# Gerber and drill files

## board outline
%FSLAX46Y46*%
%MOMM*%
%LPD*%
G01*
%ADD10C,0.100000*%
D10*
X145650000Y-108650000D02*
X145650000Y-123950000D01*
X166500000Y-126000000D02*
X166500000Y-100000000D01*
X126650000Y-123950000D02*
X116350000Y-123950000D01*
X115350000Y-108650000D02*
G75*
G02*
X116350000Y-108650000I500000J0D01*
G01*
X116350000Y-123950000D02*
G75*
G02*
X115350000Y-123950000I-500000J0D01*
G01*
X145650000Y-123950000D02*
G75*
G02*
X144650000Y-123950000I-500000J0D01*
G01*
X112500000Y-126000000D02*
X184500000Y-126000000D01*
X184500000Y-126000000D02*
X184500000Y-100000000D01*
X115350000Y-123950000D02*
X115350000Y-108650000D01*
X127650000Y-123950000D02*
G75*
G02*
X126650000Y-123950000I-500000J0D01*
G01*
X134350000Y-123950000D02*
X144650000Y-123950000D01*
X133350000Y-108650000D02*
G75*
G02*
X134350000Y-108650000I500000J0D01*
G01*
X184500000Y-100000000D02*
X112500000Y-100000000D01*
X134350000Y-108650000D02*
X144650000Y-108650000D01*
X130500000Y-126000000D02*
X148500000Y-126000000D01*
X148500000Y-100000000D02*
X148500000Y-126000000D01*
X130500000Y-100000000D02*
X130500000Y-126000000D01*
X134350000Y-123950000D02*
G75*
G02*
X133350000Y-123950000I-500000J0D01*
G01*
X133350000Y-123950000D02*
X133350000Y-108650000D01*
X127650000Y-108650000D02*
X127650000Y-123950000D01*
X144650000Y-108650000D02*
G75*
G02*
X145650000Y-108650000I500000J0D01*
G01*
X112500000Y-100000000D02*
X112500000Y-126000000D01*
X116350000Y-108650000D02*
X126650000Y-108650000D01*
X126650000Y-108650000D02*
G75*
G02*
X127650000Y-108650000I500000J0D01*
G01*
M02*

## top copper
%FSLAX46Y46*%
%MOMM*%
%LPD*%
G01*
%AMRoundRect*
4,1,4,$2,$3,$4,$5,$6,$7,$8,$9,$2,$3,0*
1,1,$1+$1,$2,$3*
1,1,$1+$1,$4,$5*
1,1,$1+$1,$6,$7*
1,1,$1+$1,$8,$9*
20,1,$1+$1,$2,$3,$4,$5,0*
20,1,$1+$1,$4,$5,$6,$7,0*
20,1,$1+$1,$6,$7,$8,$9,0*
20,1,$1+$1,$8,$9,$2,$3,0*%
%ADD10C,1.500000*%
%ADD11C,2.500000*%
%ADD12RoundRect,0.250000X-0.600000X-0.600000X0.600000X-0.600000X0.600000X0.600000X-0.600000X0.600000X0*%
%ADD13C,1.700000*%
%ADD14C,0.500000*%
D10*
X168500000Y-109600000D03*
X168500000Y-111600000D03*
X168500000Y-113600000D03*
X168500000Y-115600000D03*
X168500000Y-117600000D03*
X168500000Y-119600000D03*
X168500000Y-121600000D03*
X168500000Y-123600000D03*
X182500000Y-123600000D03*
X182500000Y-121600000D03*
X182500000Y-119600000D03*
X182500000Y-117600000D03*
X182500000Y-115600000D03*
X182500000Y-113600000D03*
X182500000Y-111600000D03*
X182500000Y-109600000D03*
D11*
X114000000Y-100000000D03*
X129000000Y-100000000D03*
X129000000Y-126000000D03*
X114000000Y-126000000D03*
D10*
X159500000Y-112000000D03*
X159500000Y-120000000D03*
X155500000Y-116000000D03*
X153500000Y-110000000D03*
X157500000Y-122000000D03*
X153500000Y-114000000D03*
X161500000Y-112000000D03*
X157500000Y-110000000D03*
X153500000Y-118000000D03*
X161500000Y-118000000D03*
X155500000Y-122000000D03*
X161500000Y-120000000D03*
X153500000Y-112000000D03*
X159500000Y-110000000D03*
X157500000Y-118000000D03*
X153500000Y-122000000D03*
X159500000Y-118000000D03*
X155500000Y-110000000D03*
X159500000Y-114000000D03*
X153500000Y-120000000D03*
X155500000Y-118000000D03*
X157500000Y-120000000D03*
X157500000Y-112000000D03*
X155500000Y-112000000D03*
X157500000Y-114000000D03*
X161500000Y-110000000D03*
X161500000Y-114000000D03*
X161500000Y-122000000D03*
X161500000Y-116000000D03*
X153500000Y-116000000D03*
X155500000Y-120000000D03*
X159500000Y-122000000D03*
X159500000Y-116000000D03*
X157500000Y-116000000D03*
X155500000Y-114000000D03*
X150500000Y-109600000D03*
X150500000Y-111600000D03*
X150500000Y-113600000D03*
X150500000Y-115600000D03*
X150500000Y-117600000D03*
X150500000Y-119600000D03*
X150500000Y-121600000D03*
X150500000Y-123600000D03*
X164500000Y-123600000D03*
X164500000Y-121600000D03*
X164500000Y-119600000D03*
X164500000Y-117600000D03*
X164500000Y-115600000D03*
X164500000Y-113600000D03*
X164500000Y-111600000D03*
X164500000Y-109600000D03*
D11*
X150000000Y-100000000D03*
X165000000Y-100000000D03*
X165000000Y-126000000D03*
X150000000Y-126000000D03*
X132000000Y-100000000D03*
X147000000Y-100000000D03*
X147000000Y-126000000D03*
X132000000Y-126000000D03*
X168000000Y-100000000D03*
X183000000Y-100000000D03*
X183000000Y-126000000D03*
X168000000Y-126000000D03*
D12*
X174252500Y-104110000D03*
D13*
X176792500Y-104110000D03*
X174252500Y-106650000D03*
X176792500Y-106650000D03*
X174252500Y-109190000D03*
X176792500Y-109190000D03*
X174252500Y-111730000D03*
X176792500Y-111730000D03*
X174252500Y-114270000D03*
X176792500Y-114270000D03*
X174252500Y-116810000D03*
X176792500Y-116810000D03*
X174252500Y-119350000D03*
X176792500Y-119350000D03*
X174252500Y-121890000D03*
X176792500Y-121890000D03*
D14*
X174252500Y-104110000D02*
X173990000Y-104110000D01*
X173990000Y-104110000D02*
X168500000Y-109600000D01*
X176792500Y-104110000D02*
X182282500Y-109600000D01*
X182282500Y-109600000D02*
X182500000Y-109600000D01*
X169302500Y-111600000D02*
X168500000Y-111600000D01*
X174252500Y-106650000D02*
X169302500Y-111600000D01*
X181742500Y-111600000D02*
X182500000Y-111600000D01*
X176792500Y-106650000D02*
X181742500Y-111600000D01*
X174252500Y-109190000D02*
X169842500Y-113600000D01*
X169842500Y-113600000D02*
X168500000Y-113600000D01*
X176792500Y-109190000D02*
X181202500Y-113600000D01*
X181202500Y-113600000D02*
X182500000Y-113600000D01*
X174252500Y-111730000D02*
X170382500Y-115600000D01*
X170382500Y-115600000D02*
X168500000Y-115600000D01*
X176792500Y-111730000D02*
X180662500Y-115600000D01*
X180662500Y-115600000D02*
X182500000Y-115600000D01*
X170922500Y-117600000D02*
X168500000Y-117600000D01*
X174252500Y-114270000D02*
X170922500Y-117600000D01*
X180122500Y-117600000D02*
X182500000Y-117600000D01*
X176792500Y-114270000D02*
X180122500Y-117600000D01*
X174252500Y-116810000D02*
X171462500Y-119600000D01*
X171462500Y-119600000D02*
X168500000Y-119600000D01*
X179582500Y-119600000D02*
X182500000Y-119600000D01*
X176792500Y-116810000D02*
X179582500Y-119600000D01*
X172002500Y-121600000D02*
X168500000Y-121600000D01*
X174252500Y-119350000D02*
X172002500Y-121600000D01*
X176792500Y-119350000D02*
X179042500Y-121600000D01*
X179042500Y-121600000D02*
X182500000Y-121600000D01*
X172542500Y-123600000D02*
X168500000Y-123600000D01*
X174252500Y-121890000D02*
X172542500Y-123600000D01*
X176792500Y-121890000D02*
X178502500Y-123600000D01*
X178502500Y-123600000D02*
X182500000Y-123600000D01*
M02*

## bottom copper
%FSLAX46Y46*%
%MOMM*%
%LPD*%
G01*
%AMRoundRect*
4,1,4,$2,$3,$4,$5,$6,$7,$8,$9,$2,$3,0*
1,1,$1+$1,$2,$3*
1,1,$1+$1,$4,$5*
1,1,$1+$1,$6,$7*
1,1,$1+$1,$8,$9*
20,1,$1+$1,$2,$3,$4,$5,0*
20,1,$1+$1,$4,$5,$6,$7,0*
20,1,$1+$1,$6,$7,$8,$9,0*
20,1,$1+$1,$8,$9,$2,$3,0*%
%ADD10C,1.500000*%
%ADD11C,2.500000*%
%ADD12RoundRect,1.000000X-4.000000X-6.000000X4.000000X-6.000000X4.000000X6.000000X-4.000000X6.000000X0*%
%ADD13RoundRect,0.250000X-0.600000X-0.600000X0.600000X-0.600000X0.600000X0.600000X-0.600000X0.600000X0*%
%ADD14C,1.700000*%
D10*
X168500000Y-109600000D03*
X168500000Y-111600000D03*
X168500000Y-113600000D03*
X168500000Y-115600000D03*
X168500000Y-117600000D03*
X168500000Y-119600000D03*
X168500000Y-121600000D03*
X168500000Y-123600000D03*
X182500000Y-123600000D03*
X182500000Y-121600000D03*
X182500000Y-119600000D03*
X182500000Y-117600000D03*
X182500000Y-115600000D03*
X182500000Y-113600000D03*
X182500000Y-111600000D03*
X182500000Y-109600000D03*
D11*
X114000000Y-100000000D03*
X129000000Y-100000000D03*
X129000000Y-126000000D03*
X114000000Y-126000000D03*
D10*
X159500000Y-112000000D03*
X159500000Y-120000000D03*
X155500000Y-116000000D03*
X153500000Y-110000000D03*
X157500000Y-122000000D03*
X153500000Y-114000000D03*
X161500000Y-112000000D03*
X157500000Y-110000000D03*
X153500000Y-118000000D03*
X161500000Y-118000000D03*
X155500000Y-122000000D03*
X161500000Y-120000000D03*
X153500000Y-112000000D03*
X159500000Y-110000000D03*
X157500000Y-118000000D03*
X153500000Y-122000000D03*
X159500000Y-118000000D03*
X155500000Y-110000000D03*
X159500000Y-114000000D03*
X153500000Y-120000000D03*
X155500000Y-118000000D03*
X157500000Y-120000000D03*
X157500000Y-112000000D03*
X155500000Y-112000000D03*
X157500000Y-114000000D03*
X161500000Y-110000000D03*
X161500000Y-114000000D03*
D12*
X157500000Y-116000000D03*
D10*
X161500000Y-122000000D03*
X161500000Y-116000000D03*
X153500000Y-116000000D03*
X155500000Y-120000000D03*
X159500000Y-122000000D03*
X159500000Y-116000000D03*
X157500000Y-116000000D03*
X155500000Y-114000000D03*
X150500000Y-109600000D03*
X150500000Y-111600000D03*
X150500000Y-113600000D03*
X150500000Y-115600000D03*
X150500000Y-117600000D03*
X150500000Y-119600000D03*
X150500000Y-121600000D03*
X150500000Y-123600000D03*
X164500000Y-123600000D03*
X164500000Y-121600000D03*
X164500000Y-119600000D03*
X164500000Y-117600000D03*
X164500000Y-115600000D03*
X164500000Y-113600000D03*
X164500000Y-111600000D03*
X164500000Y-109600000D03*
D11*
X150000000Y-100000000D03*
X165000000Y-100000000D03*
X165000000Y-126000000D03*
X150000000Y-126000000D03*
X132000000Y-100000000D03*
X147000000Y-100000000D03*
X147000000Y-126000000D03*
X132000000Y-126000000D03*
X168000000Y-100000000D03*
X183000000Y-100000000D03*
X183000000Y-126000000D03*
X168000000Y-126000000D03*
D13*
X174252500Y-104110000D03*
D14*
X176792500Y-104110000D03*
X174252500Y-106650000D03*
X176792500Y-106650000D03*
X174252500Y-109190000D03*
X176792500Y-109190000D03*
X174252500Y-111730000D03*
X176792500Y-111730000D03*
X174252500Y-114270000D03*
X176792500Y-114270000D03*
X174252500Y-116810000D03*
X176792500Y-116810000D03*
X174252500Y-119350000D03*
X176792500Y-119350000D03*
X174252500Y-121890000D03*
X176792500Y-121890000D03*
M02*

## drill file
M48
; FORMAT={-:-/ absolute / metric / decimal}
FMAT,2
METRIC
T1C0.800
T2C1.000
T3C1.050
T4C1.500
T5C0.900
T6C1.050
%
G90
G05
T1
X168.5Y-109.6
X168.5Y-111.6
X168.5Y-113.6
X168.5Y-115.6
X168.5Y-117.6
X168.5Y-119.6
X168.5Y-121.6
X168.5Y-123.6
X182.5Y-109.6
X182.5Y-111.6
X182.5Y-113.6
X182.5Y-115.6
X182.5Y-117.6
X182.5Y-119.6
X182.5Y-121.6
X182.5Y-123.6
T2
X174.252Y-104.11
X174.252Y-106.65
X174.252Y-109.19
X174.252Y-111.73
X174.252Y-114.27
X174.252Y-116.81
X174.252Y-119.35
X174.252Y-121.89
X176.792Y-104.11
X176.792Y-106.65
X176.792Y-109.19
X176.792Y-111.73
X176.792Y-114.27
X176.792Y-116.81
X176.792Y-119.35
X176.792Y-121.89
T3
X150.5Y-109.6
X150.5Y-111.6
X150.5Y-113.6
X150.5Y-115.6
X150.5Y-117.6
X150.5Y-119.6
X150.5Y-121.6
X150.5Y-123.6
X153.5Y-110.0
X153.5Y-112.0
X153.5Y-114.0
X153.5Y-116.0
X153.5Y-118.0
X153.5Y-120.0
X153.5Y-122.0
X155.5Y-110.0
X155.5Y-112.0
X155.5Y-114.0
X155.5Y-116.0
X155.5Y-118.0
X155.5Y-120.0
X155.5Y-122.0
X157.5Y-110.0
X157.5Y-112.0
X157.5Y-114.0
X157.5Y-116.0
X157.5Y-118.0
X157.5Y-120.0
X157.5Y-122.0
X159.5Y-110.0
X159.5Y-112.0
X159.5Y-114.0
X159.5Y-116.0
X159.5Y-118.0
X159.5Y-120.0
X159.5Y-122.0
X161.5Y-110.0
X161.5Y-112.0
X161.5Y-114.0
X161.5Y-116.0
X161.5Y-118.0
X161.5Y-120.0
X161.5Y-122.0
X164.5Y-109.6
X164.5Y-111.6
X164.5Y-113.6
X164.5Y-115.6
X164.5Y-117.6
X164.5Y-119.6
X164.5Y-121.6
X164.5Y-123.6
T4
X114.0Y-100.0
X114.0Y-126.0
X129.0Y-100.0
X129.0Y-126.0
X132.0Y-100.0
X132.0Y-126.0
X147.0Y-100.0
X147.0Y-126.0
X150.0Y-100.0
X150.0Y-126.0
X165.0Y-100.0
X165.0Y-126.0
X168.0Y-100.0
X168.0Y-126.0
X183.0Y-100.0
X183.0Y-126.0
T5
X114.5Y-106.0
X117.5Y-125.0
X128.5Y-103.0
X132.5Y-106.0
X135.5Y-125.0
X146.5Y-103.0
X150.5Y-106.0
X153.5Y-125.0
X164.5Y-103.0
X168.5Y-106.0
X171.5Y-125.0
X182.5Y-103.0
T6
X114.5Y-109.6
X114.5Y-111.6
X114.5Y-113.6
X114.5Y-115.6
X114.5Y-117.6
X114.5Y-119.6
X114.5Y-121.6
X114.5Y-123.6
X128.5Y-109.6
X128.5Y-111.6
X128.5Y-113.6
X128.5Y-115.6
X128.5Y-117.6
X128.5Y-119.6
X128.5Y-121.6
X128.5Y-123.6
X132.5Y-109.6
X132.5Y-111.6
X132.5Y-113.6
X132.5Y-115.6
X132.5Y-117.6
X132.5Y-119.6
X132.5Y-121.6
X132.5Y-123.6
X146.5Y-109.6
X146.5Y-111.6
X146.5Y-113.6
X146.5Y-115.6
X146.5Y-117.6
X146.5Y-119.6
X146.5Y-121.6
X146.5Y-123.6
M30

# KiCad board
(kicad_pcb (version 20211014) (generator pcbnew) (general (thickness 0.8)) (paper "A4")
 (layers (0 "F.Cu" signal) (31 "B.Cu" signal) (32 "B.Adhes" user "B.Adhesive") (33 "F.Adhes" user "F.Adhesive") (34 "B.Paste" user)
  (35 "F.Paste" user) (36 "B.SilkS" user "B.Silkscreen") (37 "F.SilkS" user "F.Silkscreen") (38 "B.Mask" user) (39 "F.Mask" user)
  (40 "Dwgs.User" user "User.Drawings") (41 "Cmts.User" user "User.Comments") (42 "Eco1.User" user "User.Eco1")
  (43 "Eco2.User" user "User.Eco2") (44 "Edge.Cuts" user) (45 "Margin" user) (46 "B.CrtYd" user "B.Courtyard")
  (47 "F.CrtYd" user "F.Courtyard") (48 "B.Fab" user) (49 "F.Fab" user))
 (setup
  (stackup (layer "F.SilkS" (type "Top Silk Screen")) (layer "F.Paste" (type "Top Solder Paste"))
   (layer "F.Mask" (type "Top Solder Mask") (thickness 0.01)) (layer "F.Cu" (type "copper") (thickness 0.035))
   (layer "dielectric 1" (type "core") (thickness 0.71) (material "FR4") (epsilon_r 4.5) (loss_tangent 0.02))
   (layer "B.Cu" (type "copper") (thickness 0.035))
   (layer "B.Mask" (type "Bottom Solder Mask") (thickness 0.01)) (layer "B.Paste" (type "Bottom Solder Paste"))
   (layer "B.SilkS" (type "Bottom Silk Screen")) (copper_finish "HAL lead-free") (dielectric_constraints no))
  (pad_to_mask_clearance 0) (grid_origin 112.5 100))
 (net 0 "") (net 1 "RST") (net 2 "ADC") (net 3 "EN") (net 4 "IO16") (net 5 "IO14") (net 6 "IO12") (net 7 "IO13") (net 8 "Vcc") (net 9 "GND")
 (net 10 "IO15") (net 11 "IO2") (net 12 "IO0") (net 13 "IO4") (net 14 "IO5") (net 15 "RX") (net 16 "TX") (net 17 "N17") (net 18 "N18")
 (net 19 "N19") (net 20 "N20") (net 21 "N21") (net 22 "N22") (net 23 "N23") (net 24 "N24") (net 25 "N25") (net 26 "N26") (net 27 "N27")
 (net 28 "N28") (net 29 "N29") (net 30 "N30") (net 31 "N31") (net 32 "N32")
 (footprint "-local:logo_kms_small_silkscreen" (layer "F.Cu") (at 153 104.474422)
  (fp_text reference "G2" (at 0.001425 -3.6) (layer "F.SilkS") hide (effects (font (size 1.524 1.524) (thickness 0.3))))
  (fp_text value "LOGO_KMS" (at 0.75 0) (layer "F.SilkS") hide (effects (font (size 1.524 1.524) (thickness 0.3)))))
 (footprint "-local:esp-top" (layer "F.Cu") (at 166.5 100)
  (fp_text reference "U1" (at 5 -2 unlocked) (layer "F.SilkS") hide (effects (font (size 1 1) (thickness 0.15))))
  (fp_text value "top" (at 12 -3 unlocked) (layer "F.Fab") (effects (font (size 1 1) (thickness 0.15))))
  (pad "1" thru_hole circle (at 2 9.6) (size 1.5 1.5) (drill 0.8) (layers *.Cu *.Mask) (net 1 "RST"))
  (pad "2" thru_hole circle (at 2 11.6) (size 1.5 1.5) (drill 0.8) (layers *.Cu *.Mask) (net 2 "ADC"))
  (pad "3" thru_hole circle (at 2 13.6) (size 1.5 1.5) (drill 0.8) (layers *.Cu *.Mask) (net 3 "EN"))
  (pad "4" thru_hole circle (at 2 15.6) (size 1.5 1.5) (drill 0.8) (layers *.Cu *.Mask) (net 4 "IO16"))
  (pad "5" thru_hole circle (at 2 17.6) (size 1.5 1.5) (drill 0.8) (layers *.Cu *.Mask) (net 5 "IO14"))
  (pad "6" thru_hole circle (at 2 19.6) (size 1.5 1.5) (drill 0.8) (layers *.Cu *.Mask) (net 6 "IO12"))
  (pad "7" thru_hole circle (at 2 21.6) (size 1.5 1.5) (drill 0.8) (layers *.Cu *.Mask) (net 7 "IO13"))
  (pad "8" thru_hole circle (at 2 23.6) (size 1.5 1.5) (drill 0.8) (layers *.Cu *.Mask) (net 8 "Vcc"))
  (pad "9" thru_hole circle (at 16 23.6) (size 1.5 1.5) (drill 0.8) (layers *.Cu *.Mask) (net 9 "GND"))
  (pad "10" thru_hole circle (at 16 21.6) (size 1.5 1.5) (drill 0.8) (layers *.Cu *.Mask) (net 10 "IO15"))
  (pad "11" thru_hole circle (at 16 19.6) (size 1.5 1.5) (drill 0.8) (layers *.Cu *.Mask) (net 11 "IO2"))
  (pad "12" thru_hole circle (at 16 17.6) (size 1.5 1.5) (drill 0.8) (layers *.Cu *.Mask) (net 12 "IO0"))
  (pad "13" thru_hole circle (at 16 15.6) (size 1.5 1.5) (drill 0.8) (layers *.Cu *.Mask) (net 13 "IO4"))
  (pad "14" thru_hole circle (at 16 13.6) (size 1.5 1.5) (drill 0.8) (layers *.Cu *.Mask) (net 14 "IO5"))
  (pad "15" thru_hole circle (at 16 11.6) (size 1.5 1.5) (drill 0.8) (layers *.Cu *.Mask) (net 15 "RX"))
  (pad "16" thru_hole circle (at 16 9.6) (size 1.5 1.5) (drill 0.8) (layers *.Cu *.Mask) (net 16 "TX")))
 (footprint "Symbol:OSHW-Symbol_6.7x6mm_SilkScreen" (layer "F.Cu") (at 161 104.5)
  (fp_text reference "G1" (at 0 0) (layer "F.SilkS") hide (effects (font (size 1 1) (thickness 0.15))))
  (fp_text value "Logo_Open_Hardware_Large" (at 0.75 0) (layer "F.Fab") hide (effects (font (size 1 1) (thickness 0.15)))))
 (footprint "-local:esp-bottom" (layer "F.Cu") (at 112.5 100)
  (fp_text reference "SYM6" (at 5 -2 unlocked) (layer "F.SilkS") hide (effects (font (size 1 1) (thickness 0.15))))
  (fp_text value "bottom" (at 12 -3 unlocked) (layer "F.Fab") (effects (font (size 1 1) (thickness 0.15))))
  (pad "" np_thru_hole circle (at 2 23.6) (size 1.05 1.05) (drill 1.05) (layers F&B.Cu *.Mask))
  (pad "" np_thru_hole circle (at 16 19.6) (size 1.05 1.05) (drill 1.05) (layers F&B.Cu *.Mask))
  (pad "" np_thru_hole circle (at 2 13.6) (size 1.05 1.05) (drill 1.05) (layers F&B.Cu *.Mask))
  (pad "" np_thru_hole circle (at 2 11.6) (size 1.05 1.05) (drill 1.05) (layers F&B.Cu *.Mask))
  (pad "" np_thru_hole circle (at 2 15.6) (size 1.05 1.05) (drill 1.05) (layers F&B.Cu *.Mask))
  (pad "" np_thru_hole circle (at 16 9.6) (size 1.05 1.05) (drill 1.05) (layers F&B.Cu *.Mask))
  (pad "" np_thru_hole circle (at 2 9.6) (size 1.05 1.05) (drill 1.05) (layers F&B.Cu *.Mask))
  (pad "" np_thru_hole circle (at 16 23.6) (size 1.05 1.05) (drill 1.05) (layers F&B.Cu *.Mask))
  (pad "" np_thru_hole circle (at 2 17.6) (size 1.05 1.05) (drill 1.05) (layers F&B.Cu *.Mask))
  (pad "" np_thru_hole circle (at 16 13.6) (size 1.05 1.05) (drill 1.05) (layers F&B.Cu *.Mask))
  (pad "" np_thru_hole circle (at 2 19.6) (size 1.05 1.05) (drill 1.05) (layers F&B.Cu *.Mask))
  (pad "" np_thru_hole circle (at 16 17.6) (size 1.05 1.05) (drill 1.05) (layers F&B.Cu *.Mask))
  (pad "" np_thru_hole circle (at 16 11.6) (size 1.05 1.05) (drill 1.05) (layers F&B.Cu *.Mask))
  (pad "" np_thru_hole circle (at 16 21.6) (size 1.05 1.05) (drill 1.05) (layers F&B.Cu *.Mask))
  (pad "" np_thru_hole circle (at 2 21.6) (size 1.05 1.05) (drill 1.05) (layers F&B.Cu *.Mask))
  (pad "" np_thru_hole circle (at 16 15.6) (size 1.05 1.05) (drill 1.05) (layers F&B.Cu *.Mask)))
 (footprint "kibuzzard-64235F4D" (layer "F.Cu") (at 157.5 124.5)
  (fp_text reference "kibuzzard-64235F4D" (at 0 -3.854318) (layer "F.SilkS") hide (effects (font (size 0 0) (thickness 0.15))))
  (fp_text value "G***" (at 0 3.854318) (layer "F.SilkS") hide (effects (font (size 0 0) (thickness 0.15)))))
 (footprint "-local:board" (layer "F.Cu") (at 112.5 100)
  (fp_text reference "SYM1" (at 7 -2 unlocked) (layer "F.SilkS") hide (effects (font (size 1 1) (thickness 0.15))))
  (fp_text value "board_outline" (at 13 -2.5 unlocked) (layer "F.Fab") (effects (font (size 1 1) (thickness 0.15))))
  (pad "" np_thru_hole circle (at 16 3) (size 0.9 0.9) (drill 0.9) (layers F&B.Cu *.Mask))
  (pad "" np_thru_hole circle (at 5 25) (size 0.9 0.9) (drill 0.9) (layers F&B.Cu *.Mask))
  (pad "" np_thru_hole circle (at 2 6) (size 0.9 0.9) (drill 0.9) (layers F&B.Cu *.Mask))
  (pad "1" thru_hole circle (at 1.5 0) (size 2.5 2.5) (drill 1.5) (layers *.Cu *.Mask))
  (pad "2" thru_hole circle (at 16.5 0) (size 2.5 2.5) (drill 1.5) (layers *.Cu *.Mask))
  (pad "3" thru_hole circle (at 16.5 26) (size 2.5 2.5) (drill 1.5) (layers *.Cu *.Mask))
  (pad "4" thru_hole circle (at 1.5 26) (size 2.5 2.5) (drill 1.5) (layers *.Cu *.Mask)))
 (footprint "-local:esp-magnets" (layer "F.Cu") (at 148.5 100)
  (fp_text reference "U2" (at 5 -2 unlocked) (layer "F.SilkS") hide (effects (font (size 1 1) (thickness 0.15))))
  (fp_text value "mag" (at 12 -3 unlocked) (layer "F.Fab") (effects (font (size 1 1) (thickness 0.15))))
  (pad "" thru_hole circle (at 11 12) (size 1.5 1.5) (drill 1.05) (layers *.Cu *.Mask))
  (pad "" thru_hole circle (at 11 20) (size 1.5 1.5) (drill 1.05) (layers *.Cu *.Mask))
  (pad "" thru_hole circle (at 7 16) (size 1.5 1.5) (drill 1.05) (layers *.Cu *.Mask))
  (pad "" thru_hole circle (at 5 10) (size 1.5 1.5) (drill 1.05) (layers *.Cu *.Mask))
  (pad "" thru_hole circle (at 9 22) (size 1.5 1.5) (drill 1.05) (layers *.Cu *.Mask))
  (pad "" thru_hole circle (at 5 14) (size 1.5 1.5) (drill 1.05) (layers *.Cu *.Mask))
  (pad "" thru_hole circle (at 13 12) (size 1.5 1.5) (drill 1.05) (layers *.Cu *.Mask))
  (pad "" thru_hole circle (at 9 10) (size 1.5 1.5) (drill 1.05) (layers *.Cu *.Mask))
  (pad "" thru_hole circle (at 5 18) (size 1.5 1.5) (drill 1.05) (layers *.Cu *.Mask))
  (pad "" thru_hole circle (at 13 18) (size 1.5 1.5) (drill 1.05) (layers *.Cu *.Mask))
  (pad "" thru_hole circle (at 7 22) (size 1.5 1.5) (drill 1.05) (layers *.Cu *.Mask))
  (pad "" thru_hole circle (at 13 20) (size 1.5 1.5) (drill 1.05) (layers *.Cu *.Mask))
  (pad "" thru_hole circle (at 5 12) (size 1.5 1.5) (drill 1.05) (layers *.Cu *.Mask))
  (pad "" thru_hole circle (at 11 10) (size 1.5 1.5) (drill 1.05) (layers *.Cu *.Mask))
  (pad "" thru_hole circle (at 9 18) (size 1.5 1.5) (drill 1.05) (layers *.Cu *.Mask))
  (pad "" thru_hole circle (at 5 22) (size 1.5 1.5) (drill 1.05) (layers *.Cu *.Mask))
  (pad "" thru_hole circle (at 11 18) (size 1.5 1.5) (drill 1.05) (layers *.Cu *.Mask))
  (pad "" thru_hole circle (at 7 10) (size 1.5 1.5) (drill 1.05) (layers *.Cu *.Mask))
  (pad "" thru_hole circle (at 11 14) (size 1.5 1.5) (drill 1.05) (layers *.Cu *.Mask))
  (pad "" thru_hole circle (at 5 20) (size 1.5 1.5) (drill 1.05) (layers *.Cu *.Mask))
  (pad "" thru_hole circle (at 7 18) (size 1.5 1.5) (drill 1.05) (layers *.Cu *.Mask))
  (pad "" thru_hole circle (at 9 20) (size 1.5 1.5) (drill 1.05) (layers *.Cu *.Mask))
  (pad "" thru_hole circle (at 9 12) (size 1.5 1.5) (drill 1.05) (layers *.Cu *.Mask))
  (pad "" thru_hole circle (at 7 12) (size 1.5 1.5) (drill 1.05) (layers *.Cu *.Mask))
  (pad "" thru_hole circle (at 9 14) (size 1.5 1.5) (drill 1.05) (layers *.Cu *.Mask))
  (pad "" thru_hole circle (at 13 10) (size 1.5 1.5) (drill 1.05) (layers *.Cu *.Mask))
  (pad "" thru_hole circle (at 13 14) (size 1.5 1.5) (drill 1.05) (layers *.Cu *.Mask))
  (pad "" smd roundrect (at 9 16) (size 10 14) (layers "B.Cu" "B.Mask") (roundrect_rratio 0.1))
  (pad "" thru_hole circle (at 13 22) (size 1.5 1.5) (drill 1.05) (layers *.Cu *.Mask))
  (pad "" thru_hole circle (at 13 16) (size 1.5 1.5) (drill 1.05) (layers *.Cu *.Mask))
  (pad "" thru_hole circle (at 5 16) (size 1.5 1.5) (drill 1.05) (layers *.Cu *.Mask))
  (pad "" thru_hole circle (at 7 20) (size 1.5 1.5) (drill 1.05) (layers *.Cu *.Mask))
  (pad "" thru_hole circle (at 11 22) (size 1.5 1.5) (drill 1.05) (layers *.Cu *.Mask))
  (pad "" thru_hole circle (at 11 16) (size 1.5 1.5) (drill 1.05) (layers *.Cu *.Mask))
  (pad "" thru_hole circle (at 9 16) (size 1.5 1.5) (drill 1.05) (layers *.Cu *.Mask))
  (pad "" thru_hole circle (at 7 14) (size 1.5 1.5) (drill 1.05) (layers *.Cu *.Mask))
  (pad "1" thru_hole circle (at 2 9.6) (size 1.5 1.5) (drill 1.05) (layers *.Cu *.Mask) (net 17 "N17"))
  (pad "2" thru_hole circle (at 2 11.6) (size 1.5 1.5) (drill 1.05) (layers *.Cu *.Mask) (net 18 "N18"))
  (pad "3" thru_hole circle (at 2 13.6) (size 1.5 1.5) (drill 1.05) (layers *.Cu *.Mask) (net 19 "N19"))
  (pad "4" thru_hole circle (at 2 15.6) (size 1.5 1.5) (drill 1.05) (layers *.Cu *.Mask) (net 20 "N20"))
  (pad "5" thru_hole circle (at 2 17.6) (size 1.5 1.5) (drill 1.05) (layers *.Cu *.Mask) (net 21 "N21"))
  (pad "6" thru_hole circle (at 2 19.6) (size 1.5 1.5) (drill 1.05) (layers *.Cu *.Mask) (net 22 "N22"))
  (pad "7" thru_hole circle (at 2 21.6) (size 1.5 1.5) (drill 1.05) (layers *.Cu *.Mask) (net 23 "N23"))
  (pad "8" thru_hole circle (at 2 23.6) (size 1.5 1.5) (drill 1.05) (layers *.Cu *.Mask) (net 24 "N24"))
  (pad "9" thru_hole circle (at 16 23.6) (size 1.5 1.5) (drill 1.05) (layers *.Cu *.Mask) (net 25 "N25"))
  (pad "10" thru_hole circle (at 16 21.6) (size 1.5 1.5) (drill 1.05) (layers *.Cu *.Mask) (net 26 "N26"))
  (pad "11" thru_hole circle (at 16 19.6) (size 1.5 1.5) (drill 1.05) (layers *.Cu *.Mask) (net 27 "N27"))
  (pad "12" thru_hole circle (at 16 17.6) (size 1.5 1.5) (drill 1.05) (layers *.Cu *.Mask) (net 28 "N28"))
  (pad "13" thru_hole circle (at 16 15.6) (size 1.5 1.5) (drill 1.05) (layers *.Cu *.Mask) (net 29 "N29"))
  (pad "14" thru_hole circle (at 16 13.6) (size 1.5 1.5) (drill 1.05) (layers *.Cu *.Mask) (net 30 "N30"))
  (pad "15" thru_hole circle (at 16 11.6) (size 1.5 1.5) (drill 1.05) (layers *.Cu *.Mask) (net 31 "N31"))
  (pad "16" thru_hole circle (at 16 9.6) (size 1.5 1.5) (drill 1.05) (layers *.Cu *.Mask) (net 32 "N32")))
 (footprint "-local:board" (layer "F.Cu") (at 148.5 100)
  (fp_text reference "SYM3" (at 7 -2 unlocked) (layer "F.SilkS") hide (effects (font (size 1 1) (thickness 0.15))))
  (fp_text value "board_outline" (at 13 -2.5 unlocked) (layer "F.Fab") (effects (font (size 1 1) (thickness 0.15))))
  (pad "" np_thru_hole circle (at 5 25) (size 0.9 0.9) (drill 0.9) (layers F&B.Cu *.Mask))
  (pad "" np_thru_hole circle (at 2 6) (size 0.9 0.9) (drill 0.9) (layers F&B.Cu *.Mask))
  (pad "" np_thru_hole circle (at 16 3) (size 0.9 0.9) (drill 0.9) (layers F&B.Cu *.Mask))
  (pad "1" thru_hole circle (at 1.5 0) (size 2.5 2.5) (drill 1.5) (layers *.Cu *.Mask))
  (pad "2" thru_hole circle (at 16.5 0) (size 2.5 2.5) (drill 1.5) (layers *.Cu *.Mask))
  (pad "3" thru_hole circle (at 16.5 26) (size 2.5 2.5) (drill 1.5) (layers *.Cu *.Mask))
  (pad "4" thru_hole circle (at 1.5 26) (size 2.5 2.5) (drill 1.5) (layers *.Cu *.Mask)))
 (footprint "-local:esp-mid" (layer "F.Cu") (at 130.5 100)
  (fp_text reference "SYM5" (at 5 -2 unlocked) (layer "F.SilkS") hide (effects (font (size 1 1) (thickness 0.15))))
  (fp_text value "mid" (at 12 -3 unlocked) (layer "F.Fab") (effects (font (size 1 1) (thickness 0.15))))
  (pad "" np_thru_hole circle (at 2 17.6) (size 1.05 1.05) (drill 1.05) (layers F&B.Cu *.Mask))
  (pad "" np_thru_hole circle (at 2 15.6) (size 1.05 1.05) (drill 1.05) (layers F&B.Cu *.Mask))
  (pad "" np_thru_hole circle (at 2 9.6) (size 1.05 1.05) (drill 1.05) (layers F&B.Cu *.Mask))
  (pad "" np_thru_hole circle (at 16 21.6) (size 1.05 1.05) (drill 1.05) (layers F&B.Cu *.Mask))
  (pad "" np_thru_hole circle (at 2 19.6) (size 1.05 1.05) (drill 1.05) (layers F&B.Cu *.Mask))
  (pad "" np_thru_hole circle (at 2 23.6) (size 1.05 1.05) (drill 1.05) (layers F&B.Cu *.Mask))
  (pad "" np_thru_hole circle (at 16 15.6) (size 1.05 1.05) (drill 1.05) (layers F&B.Cu *.Mask))
  (pad "" np_thru_hole circle (at 16 19.6) (size 1.05 1.05) (drill 1.05) (layers F&B.Cu *.Mask))
  (pad "" np_thru_hole circle (at 2 11.6) (size 1.05 1.05) (drill 1.05) (layers F&B.Cu *.Mask))
  (pad "" np_thru_hole circle (at 16 17.6) (size 1.05 1.05) (drill 1.05) (layers F&B.Cu *.Mask))
  (pad "" np_thru_hole circle (at 2 13.6) (size 1.05 1.05) (drill 1.05) (layers F&B.Cu *.Mask))
  (pad "" np_thru_hole circle (at 16 11.6) (size 1.05 1.05) (drill 1.05) (layers F&B.Cu *.Mask))
  (pad "" np_thru_hole circle (at 16 13.6) (size 1.05 1.05) (drill 1.05) (layers F&B.Cu *.Mask))
  (pad "" np_thru_hole circle (at 16 23.6) (size 1.05 1.05) (drill 1.05) (layers F&B.Cu *.Mask))
  (pad "" np_thru_hole circle (at 16 9.6) (size 1.05 1.05) (drill 1.05) (layers F&B.Cu *.Mask))
  (pad "" np_thru_hole circle (at 2 21.6) (size 1.05 1.05) (drill 1.05) (layers F&B.Cu *.Mask)))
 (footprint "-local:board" (layer "F.Cu") (at 130.5 100)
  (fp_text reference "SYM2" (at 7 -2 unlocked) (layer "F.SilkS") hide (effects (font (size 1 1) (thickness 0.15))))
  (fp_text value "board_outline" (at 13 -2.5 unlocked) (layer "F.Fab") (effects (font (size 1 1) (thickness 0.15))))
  (pad "" np_thru_hole circle (at 5 25) (size 0.9 0.9) (drill 0.9) (layers F&B.Cu *.Mask))
  (pad "" np_thru_hole circle (at 16 3) (size 0.9 0.9) (drill 0.9) (layers F&B.Cu *.Mask))
  (pad "" np_thru_hole circle (at 2 6) (size 0.9 0.9) (drill 0.9) (layers F&B.Cu *.Mask))
  (pad "1" thru_hole circle (at 1.5 0) (size 2.5 2.5) (drill 1.5) (layers *.Cu *.Mask))
  (pad "2" thru_hole circle (at 16.5 0) (size 2.5 2.5) (drill 1.5) (layers *.Cu *.Mask))
  (pad "3" thru_hole circle (at 16.5 26) (size 2.5 2.5) (drill 1.5) (layers *.Cu *.Mask))
  (pad "4" thru_hole circle (at 1.5 26) (size 2.5 2.5) (drill 1.5) (layers *.Cu *.Mask)))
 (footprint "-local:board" (layer "F.Cu") (at 166.5 100)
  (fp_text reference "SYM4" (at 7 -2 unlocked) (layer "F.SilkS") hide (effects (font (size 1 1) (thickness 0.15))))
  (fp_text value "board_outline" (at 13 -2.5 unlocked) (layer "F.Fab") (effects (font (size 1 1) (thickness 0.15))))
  (pad "" np_thru_hole circle (at 5 25) (size 0.9 0.9) (drill 0.9) (layers F&B.Cu *.Mask))
  (pad "" np_thru_hole circle (at 16 3) (size 0.9 0.9) (drill 0.9) (layers F&B.Cu *.Mask))
  (pad "" np_thru_hole circle (at 2 6) (size 0.9 0.9) (drill 0.9) (layers F&B.Cu *.Mask))
  (pad "1" thru_hole circle (at 1.5 0) (size 2.5 2.5) (drill 1.5) (layers *.Cu *.Mask))
  (pad "2" thru_hole circle (at 16.5 0) (size 2.5 2.5) (drill 1.5) (layers *.Cu *.Mask))
  (pad "3" thru_hole circle (at 16.5 26) (size 2.5 2.5) (drill 1.5) (layers *.Cu *.Mask))
  (pad "4" thru_hole circle (at 1.5 26) (size 2.5 2.5) (drill 1.5) (layers *.Cu *.Mask)))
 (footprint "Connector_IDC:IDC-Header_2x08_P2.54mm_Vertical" (layer "F.Cu") (at 174.2525 104.11)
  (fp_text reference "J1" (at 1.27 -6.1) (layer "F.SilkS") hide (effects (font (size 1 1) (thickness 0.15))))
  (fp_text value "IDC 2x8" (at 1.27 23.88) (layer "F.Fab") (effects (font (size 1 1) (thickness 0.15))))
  (pad "1" thru_hole roundrect (at 0 0) (size 1.7 1.7) (drill 1) (layers *.Cu *.Mask) (roundrect_rratio 0.147059) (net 1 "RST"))
  (pad "2" thru_hole circle (at 2.54 0) (size 1.7 1.7) (drill 1) (layers *.Cu *.Mask) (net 16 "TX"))
  (pad "3" thru_hole circle (at 0 2.54) (size 1.7 1.7) (drill 1) (layers *.Cu *.Mask) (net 2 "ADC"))
  (pad "4" thru_hole circle (at 2.54 2.54) (size 1.7 1.7) (drill 1) (layers *.Cu *.Mask) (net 15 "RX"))
  (pad "5" thru_hole circle (at 0 5.08) (size 1.7 1.7) (drill 1) (layers *.Cu *.Mask) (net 3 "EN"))
  (pad "6" thru_hole circle (at 2.54 5.08) (size 1.7 1.7) (drill 1) (layers *.Cu *.Mask) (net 14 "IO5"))
  (pad "7" thru_hole circle (at 0 7.62) (size 1.7 1.7) (drill 1) (layers *.Cu *.Mask) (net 4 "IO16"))
  (pad "8" thru_hole circle (at 2.54 7.62) (size 1.7 1.7) (drill 1) (layers *.Cu *.Mask) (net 13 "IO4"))
  (pad "9" thru_hole circle (at 0 10.16) (size 1.7 1.7) (drill 1) (layers *.Cu *.Mask) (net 5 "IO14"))
  (pad "10" thru_hole circle (at 2.54 10.16) (size 1.7 1.7) (drill 1) (layers *.Cu *.Mask) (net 12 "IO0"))
  (pad "11" thru_hole circle (at 0 12.7) (size 1.7 1.7) (drill 1) (layers *.Cu *.Mask) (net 6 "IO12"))
  (pad "12" thru_hole circle (at 2.54 12.7) (size 1.7 1.7) (drill 1) (layers *.Cu *.Mask) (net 11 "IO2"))
  (pad "13" thru_hole circle (at 0 15.24) (size 1.7 1.7) (drill 1) (layers *.Cu *.Mask) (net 7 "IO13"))
  (pad "14" thru_hole circle (at 2.54 15.24) (size 1.7 1.7) (drill 1) (layers *.Cu *.Mask) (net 10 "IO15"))
  (pad "15" thru_hole circle (at 0 17.78) (size 1.7 1.7) (drill 1) (layers *.Cu *.Mask) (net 8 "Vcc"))
  (pad "16" thru_hole circle (at 2.54 17.78) (size 1.7 1.7) (drill 1) (layers *.Cu *.Mask) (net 9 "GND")))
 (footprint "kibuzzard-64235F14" (layer "B.Cu") (at 121.5 125 180)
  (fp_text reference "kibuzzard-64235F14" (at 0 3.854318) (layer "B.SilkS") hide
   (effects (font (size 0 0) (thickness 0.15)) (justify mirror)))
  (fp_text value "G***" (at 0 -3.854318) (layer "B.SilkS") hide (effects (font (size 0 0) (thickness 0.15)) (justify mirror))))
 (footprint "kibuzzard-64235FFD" (layer "B.Cu") (at 180.5 113 -90)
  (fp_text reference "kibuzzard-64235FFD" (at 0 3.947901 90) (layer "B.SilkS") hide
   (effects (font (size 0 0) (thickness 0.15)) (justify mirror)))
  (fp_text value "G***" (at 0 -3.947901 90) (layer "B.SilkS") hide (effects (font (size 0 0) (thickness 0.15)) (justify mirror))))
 (gr_line (start 145.65 108.65) (end 145.65 123.95) (layer "Edge.Cuts") (width 0.1))
 (gr_line (start 166.5 126) (end 166.5 100) (layer "Edge.Cuts") (width 0.1))
 (gr_line (start 126.65 123.95) (end 116.35 123.95) (layer "Edge.Cuts") (width 0.1))
 (gr_arc (start 115.35 108.65) (mid 115.85 108.15) (end 116.35 108.65) (layer "Edge.Cuts") (width 0.1))
 (gr_arc (start 116.35 123.95) (mid 115.85 124.45) (end 115.35 123.95) (layer "Edge.Cuts") (width 0.1))
 (gr_arc (start 145.65 123.95) (mid 145.15 124.45) (end 144.65 123.95) (layer "Edge.Cuts") (width 0.1))
 (gr_line (start 112.5 126) (end 184.5 126) (layer "Edge.Cuts") (width 0.1))
 (gr_line (start 184.5 126) (end 184.5 100) (layer "Edge.Cuts") (width 0.1))
 (gr_line (start 115.35 123.95) (end 115.35 108.65) (layer "Edge.Cuts") (width 0.1))
 (gr_arc (start 127.65 123.95) (mid 127.15 124.45) (end 126.65 123.95) (layer "Edge.Cuts") (width 0.1))
 (gr_line (start 134.35 123.95) (end 144.65 123.95) (layer "Edge.Cuts") (width 0.1))
 (gr_arc (start 133.35 108.65) (mid 133.85 108.15) (end 134.35 108.65) (layer "Edge.Cuts") (width 0.1))
 (gr_line (start 184.5 100) (end 112.5 100) (layer "Edge.Cuts") (width 0.1))
 (gr_line (start 134.35 108.65) (end 144.65 108.65) (layer "Edge.Cuts") (width 0.1))
 (gr_line (start 130.5 126) (end 148.5 126) (layer "Edge.Cuts") (width 0.1))
 (gr_line (start 148.5 100) (end 148.5 126) (layer "Edge.Cuts") (width 0.1))
 (gr_line (start 130.5 100) (end 130.5 126) (layer "Edge.Cuts") (width 0.1))
 (gr_arc (start 134.35 123.95) (mid 133.85 124.45) (end 133.35 123.95) (layer "Edge.Cuts") (width 0.1))
 (gr_line (start 133.35 123.95) (end 133.35 108.65) (layer "Edge.Cuts") (width 0.1))
 (gr_line (start 127.65 108.65) (end 127.65 123.95) (layer "Edge.Cuts") (width 0.1))
 (gr_arc (start 144.65 108.65) (mid 145.15 108.15) (end 145.65 108.65) (layer "Edge.Cuts") (width 0.1))
 (gr_line (start 112.5 100) (end 112.5 126) (layer "Edge.Cuts") (width 0.1))
 (gr_line (start 116.35 108.65) (end 126.65 108.65) (layer "Edge.Cuts") (width 0.1))
 (gr_arc (start 126.65 108.65) (mid 127.15 108.15) (end 127.65 108.65) (layer "Edge.Cuts") (width 0.1))
 (segment (start 174.2525 104.11) (end 173.99 104.11) (width 0.5) (layer "F.Cu") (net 1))
 (segment (start 173.99 104.11) (end 168.5 109.6) (width 0.5) (layer "F.Cu") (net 1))
 (segment (start 176.7925 104.11) (end 182.2825 109.6) (width 0.5) (layer "F.Cu") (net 16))
 (segment (start 182.2825 109.6) (end 182.5 109.6) (width 0.5) (layer "F.Cu") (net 16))
 (segment (start 169.3025 111.6) (end 168.5 111.6) (width 0.5) (layer "F.Cu") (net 2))
 (segment (start 174.2525 106.65) (end 169.3025 111.6) (width 0.5) (layer "F.Cu") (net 2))
 (segment (start 181.7425 111.6) (end 182.5 111.6) (width 0.5) (layer "F.Cu") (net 15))
 (segment (start 176.7925 106.65) (end 181.7425 111.6) (width 0.5) (layer "F.Cu") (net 15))
 (segment (start 174.2525 109.19) (end 169.8425 113.6) (width 0.5) (layer "F.Cu") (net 3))
 (segment (start 169.8425 113.6) (end 168.5 113.6) (width 0.5) (layer "F.Cu") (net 3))
 (segment (start 176.7925 109.19) (end 181.2025 113.6) (width 0.5) (layer "F.Cu") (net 14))
 (segment (start 181.2025 113.6) (end 182.5 113.6) (width 0.5) (layer "F.Cu") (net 14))
 (segment (start 174.2525 111.73) (end 170.3825 115.6) (width 0.5) (layer "F.Cu") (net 4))
 (segment (start 170.3825 115.6) (end 168.5 115.6) (width 0.5) (layer "F.Cu") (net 4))
 (segment (start 176.7925 111.73) (end 180.6625 115.6) (width 0.5) (layer "F.Cu") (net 13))
 (segment (start 180.6625 115.6) (end 182.5 115.6) (width 0.5) (layer "F.Cu") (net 13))
 (segment (start 170.9225 117.6) (end 168.5 117.6) (width 0.5) (layer "F.Cu") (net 5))
 (segment (start 174.2525 114.27) (end 170.9225 117.6) (width 0.5) (layer "F.Cu") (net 5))
 (segment (start 180.1225 117.6) (end 182.5 117.6) (width 0.5) (layer "F.Cu") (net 12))
 (segment (start 176.7925 114.27) (end 180.1225 117.6) (width 0.5) (layer "F.Cu") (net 12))
 (segment (start 174.2525 116.81) (end 171.4625 119.6) (width 0.5) (layer "F.Cu") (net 6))
 (segment (start 171.4625 119.6) (end 168.5 119.6) (width 0.5) (layer "F.Cu") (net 6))
 (segment (start 179.5825 119.6) (end 182.5 119.6) (width 0.5) (layer "F.Cu") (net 11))
 (segment (start 176.7925 116.81) (end 179.5825 119.6) (width 0.5) (layer "F.Cu") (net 11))
 (segment (start 172.0025 121.6) (end 168.5 121.6) (width 0.5) (layer "F.Cu") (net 7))
 (segment (start 174.2525 119.35) (end 172.0025 121.6) (width 0.5) (layer "F.Cu") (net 7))
 (segment (start 176.7925 119.35) (end 179.0425 121.6) (width 0.5) (layer "F.Cu") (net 10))
 (segment (start 179.0425 121.6) (end 182.5 121.6) (width 0.5) (layer "F.Cu") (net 10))
 (segment (start 172.5425 123.6) (end 168.5 123.6) (width 0.5) (layer "F.Cu") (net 8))
 (segment (start 174.2525 121.89) (end 172.5425 123.6) (width 0.5) (layer "F.Cu") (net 8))
 (segment (start 176.7925 121.89) (end 178.5025 123.6) (width 0.5) (layer "F.Cu") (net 9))
 (segment (start 178.5025 123.6) (end 182.5 123.6) (width 0.5) (layer "F.Cu") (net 9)))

